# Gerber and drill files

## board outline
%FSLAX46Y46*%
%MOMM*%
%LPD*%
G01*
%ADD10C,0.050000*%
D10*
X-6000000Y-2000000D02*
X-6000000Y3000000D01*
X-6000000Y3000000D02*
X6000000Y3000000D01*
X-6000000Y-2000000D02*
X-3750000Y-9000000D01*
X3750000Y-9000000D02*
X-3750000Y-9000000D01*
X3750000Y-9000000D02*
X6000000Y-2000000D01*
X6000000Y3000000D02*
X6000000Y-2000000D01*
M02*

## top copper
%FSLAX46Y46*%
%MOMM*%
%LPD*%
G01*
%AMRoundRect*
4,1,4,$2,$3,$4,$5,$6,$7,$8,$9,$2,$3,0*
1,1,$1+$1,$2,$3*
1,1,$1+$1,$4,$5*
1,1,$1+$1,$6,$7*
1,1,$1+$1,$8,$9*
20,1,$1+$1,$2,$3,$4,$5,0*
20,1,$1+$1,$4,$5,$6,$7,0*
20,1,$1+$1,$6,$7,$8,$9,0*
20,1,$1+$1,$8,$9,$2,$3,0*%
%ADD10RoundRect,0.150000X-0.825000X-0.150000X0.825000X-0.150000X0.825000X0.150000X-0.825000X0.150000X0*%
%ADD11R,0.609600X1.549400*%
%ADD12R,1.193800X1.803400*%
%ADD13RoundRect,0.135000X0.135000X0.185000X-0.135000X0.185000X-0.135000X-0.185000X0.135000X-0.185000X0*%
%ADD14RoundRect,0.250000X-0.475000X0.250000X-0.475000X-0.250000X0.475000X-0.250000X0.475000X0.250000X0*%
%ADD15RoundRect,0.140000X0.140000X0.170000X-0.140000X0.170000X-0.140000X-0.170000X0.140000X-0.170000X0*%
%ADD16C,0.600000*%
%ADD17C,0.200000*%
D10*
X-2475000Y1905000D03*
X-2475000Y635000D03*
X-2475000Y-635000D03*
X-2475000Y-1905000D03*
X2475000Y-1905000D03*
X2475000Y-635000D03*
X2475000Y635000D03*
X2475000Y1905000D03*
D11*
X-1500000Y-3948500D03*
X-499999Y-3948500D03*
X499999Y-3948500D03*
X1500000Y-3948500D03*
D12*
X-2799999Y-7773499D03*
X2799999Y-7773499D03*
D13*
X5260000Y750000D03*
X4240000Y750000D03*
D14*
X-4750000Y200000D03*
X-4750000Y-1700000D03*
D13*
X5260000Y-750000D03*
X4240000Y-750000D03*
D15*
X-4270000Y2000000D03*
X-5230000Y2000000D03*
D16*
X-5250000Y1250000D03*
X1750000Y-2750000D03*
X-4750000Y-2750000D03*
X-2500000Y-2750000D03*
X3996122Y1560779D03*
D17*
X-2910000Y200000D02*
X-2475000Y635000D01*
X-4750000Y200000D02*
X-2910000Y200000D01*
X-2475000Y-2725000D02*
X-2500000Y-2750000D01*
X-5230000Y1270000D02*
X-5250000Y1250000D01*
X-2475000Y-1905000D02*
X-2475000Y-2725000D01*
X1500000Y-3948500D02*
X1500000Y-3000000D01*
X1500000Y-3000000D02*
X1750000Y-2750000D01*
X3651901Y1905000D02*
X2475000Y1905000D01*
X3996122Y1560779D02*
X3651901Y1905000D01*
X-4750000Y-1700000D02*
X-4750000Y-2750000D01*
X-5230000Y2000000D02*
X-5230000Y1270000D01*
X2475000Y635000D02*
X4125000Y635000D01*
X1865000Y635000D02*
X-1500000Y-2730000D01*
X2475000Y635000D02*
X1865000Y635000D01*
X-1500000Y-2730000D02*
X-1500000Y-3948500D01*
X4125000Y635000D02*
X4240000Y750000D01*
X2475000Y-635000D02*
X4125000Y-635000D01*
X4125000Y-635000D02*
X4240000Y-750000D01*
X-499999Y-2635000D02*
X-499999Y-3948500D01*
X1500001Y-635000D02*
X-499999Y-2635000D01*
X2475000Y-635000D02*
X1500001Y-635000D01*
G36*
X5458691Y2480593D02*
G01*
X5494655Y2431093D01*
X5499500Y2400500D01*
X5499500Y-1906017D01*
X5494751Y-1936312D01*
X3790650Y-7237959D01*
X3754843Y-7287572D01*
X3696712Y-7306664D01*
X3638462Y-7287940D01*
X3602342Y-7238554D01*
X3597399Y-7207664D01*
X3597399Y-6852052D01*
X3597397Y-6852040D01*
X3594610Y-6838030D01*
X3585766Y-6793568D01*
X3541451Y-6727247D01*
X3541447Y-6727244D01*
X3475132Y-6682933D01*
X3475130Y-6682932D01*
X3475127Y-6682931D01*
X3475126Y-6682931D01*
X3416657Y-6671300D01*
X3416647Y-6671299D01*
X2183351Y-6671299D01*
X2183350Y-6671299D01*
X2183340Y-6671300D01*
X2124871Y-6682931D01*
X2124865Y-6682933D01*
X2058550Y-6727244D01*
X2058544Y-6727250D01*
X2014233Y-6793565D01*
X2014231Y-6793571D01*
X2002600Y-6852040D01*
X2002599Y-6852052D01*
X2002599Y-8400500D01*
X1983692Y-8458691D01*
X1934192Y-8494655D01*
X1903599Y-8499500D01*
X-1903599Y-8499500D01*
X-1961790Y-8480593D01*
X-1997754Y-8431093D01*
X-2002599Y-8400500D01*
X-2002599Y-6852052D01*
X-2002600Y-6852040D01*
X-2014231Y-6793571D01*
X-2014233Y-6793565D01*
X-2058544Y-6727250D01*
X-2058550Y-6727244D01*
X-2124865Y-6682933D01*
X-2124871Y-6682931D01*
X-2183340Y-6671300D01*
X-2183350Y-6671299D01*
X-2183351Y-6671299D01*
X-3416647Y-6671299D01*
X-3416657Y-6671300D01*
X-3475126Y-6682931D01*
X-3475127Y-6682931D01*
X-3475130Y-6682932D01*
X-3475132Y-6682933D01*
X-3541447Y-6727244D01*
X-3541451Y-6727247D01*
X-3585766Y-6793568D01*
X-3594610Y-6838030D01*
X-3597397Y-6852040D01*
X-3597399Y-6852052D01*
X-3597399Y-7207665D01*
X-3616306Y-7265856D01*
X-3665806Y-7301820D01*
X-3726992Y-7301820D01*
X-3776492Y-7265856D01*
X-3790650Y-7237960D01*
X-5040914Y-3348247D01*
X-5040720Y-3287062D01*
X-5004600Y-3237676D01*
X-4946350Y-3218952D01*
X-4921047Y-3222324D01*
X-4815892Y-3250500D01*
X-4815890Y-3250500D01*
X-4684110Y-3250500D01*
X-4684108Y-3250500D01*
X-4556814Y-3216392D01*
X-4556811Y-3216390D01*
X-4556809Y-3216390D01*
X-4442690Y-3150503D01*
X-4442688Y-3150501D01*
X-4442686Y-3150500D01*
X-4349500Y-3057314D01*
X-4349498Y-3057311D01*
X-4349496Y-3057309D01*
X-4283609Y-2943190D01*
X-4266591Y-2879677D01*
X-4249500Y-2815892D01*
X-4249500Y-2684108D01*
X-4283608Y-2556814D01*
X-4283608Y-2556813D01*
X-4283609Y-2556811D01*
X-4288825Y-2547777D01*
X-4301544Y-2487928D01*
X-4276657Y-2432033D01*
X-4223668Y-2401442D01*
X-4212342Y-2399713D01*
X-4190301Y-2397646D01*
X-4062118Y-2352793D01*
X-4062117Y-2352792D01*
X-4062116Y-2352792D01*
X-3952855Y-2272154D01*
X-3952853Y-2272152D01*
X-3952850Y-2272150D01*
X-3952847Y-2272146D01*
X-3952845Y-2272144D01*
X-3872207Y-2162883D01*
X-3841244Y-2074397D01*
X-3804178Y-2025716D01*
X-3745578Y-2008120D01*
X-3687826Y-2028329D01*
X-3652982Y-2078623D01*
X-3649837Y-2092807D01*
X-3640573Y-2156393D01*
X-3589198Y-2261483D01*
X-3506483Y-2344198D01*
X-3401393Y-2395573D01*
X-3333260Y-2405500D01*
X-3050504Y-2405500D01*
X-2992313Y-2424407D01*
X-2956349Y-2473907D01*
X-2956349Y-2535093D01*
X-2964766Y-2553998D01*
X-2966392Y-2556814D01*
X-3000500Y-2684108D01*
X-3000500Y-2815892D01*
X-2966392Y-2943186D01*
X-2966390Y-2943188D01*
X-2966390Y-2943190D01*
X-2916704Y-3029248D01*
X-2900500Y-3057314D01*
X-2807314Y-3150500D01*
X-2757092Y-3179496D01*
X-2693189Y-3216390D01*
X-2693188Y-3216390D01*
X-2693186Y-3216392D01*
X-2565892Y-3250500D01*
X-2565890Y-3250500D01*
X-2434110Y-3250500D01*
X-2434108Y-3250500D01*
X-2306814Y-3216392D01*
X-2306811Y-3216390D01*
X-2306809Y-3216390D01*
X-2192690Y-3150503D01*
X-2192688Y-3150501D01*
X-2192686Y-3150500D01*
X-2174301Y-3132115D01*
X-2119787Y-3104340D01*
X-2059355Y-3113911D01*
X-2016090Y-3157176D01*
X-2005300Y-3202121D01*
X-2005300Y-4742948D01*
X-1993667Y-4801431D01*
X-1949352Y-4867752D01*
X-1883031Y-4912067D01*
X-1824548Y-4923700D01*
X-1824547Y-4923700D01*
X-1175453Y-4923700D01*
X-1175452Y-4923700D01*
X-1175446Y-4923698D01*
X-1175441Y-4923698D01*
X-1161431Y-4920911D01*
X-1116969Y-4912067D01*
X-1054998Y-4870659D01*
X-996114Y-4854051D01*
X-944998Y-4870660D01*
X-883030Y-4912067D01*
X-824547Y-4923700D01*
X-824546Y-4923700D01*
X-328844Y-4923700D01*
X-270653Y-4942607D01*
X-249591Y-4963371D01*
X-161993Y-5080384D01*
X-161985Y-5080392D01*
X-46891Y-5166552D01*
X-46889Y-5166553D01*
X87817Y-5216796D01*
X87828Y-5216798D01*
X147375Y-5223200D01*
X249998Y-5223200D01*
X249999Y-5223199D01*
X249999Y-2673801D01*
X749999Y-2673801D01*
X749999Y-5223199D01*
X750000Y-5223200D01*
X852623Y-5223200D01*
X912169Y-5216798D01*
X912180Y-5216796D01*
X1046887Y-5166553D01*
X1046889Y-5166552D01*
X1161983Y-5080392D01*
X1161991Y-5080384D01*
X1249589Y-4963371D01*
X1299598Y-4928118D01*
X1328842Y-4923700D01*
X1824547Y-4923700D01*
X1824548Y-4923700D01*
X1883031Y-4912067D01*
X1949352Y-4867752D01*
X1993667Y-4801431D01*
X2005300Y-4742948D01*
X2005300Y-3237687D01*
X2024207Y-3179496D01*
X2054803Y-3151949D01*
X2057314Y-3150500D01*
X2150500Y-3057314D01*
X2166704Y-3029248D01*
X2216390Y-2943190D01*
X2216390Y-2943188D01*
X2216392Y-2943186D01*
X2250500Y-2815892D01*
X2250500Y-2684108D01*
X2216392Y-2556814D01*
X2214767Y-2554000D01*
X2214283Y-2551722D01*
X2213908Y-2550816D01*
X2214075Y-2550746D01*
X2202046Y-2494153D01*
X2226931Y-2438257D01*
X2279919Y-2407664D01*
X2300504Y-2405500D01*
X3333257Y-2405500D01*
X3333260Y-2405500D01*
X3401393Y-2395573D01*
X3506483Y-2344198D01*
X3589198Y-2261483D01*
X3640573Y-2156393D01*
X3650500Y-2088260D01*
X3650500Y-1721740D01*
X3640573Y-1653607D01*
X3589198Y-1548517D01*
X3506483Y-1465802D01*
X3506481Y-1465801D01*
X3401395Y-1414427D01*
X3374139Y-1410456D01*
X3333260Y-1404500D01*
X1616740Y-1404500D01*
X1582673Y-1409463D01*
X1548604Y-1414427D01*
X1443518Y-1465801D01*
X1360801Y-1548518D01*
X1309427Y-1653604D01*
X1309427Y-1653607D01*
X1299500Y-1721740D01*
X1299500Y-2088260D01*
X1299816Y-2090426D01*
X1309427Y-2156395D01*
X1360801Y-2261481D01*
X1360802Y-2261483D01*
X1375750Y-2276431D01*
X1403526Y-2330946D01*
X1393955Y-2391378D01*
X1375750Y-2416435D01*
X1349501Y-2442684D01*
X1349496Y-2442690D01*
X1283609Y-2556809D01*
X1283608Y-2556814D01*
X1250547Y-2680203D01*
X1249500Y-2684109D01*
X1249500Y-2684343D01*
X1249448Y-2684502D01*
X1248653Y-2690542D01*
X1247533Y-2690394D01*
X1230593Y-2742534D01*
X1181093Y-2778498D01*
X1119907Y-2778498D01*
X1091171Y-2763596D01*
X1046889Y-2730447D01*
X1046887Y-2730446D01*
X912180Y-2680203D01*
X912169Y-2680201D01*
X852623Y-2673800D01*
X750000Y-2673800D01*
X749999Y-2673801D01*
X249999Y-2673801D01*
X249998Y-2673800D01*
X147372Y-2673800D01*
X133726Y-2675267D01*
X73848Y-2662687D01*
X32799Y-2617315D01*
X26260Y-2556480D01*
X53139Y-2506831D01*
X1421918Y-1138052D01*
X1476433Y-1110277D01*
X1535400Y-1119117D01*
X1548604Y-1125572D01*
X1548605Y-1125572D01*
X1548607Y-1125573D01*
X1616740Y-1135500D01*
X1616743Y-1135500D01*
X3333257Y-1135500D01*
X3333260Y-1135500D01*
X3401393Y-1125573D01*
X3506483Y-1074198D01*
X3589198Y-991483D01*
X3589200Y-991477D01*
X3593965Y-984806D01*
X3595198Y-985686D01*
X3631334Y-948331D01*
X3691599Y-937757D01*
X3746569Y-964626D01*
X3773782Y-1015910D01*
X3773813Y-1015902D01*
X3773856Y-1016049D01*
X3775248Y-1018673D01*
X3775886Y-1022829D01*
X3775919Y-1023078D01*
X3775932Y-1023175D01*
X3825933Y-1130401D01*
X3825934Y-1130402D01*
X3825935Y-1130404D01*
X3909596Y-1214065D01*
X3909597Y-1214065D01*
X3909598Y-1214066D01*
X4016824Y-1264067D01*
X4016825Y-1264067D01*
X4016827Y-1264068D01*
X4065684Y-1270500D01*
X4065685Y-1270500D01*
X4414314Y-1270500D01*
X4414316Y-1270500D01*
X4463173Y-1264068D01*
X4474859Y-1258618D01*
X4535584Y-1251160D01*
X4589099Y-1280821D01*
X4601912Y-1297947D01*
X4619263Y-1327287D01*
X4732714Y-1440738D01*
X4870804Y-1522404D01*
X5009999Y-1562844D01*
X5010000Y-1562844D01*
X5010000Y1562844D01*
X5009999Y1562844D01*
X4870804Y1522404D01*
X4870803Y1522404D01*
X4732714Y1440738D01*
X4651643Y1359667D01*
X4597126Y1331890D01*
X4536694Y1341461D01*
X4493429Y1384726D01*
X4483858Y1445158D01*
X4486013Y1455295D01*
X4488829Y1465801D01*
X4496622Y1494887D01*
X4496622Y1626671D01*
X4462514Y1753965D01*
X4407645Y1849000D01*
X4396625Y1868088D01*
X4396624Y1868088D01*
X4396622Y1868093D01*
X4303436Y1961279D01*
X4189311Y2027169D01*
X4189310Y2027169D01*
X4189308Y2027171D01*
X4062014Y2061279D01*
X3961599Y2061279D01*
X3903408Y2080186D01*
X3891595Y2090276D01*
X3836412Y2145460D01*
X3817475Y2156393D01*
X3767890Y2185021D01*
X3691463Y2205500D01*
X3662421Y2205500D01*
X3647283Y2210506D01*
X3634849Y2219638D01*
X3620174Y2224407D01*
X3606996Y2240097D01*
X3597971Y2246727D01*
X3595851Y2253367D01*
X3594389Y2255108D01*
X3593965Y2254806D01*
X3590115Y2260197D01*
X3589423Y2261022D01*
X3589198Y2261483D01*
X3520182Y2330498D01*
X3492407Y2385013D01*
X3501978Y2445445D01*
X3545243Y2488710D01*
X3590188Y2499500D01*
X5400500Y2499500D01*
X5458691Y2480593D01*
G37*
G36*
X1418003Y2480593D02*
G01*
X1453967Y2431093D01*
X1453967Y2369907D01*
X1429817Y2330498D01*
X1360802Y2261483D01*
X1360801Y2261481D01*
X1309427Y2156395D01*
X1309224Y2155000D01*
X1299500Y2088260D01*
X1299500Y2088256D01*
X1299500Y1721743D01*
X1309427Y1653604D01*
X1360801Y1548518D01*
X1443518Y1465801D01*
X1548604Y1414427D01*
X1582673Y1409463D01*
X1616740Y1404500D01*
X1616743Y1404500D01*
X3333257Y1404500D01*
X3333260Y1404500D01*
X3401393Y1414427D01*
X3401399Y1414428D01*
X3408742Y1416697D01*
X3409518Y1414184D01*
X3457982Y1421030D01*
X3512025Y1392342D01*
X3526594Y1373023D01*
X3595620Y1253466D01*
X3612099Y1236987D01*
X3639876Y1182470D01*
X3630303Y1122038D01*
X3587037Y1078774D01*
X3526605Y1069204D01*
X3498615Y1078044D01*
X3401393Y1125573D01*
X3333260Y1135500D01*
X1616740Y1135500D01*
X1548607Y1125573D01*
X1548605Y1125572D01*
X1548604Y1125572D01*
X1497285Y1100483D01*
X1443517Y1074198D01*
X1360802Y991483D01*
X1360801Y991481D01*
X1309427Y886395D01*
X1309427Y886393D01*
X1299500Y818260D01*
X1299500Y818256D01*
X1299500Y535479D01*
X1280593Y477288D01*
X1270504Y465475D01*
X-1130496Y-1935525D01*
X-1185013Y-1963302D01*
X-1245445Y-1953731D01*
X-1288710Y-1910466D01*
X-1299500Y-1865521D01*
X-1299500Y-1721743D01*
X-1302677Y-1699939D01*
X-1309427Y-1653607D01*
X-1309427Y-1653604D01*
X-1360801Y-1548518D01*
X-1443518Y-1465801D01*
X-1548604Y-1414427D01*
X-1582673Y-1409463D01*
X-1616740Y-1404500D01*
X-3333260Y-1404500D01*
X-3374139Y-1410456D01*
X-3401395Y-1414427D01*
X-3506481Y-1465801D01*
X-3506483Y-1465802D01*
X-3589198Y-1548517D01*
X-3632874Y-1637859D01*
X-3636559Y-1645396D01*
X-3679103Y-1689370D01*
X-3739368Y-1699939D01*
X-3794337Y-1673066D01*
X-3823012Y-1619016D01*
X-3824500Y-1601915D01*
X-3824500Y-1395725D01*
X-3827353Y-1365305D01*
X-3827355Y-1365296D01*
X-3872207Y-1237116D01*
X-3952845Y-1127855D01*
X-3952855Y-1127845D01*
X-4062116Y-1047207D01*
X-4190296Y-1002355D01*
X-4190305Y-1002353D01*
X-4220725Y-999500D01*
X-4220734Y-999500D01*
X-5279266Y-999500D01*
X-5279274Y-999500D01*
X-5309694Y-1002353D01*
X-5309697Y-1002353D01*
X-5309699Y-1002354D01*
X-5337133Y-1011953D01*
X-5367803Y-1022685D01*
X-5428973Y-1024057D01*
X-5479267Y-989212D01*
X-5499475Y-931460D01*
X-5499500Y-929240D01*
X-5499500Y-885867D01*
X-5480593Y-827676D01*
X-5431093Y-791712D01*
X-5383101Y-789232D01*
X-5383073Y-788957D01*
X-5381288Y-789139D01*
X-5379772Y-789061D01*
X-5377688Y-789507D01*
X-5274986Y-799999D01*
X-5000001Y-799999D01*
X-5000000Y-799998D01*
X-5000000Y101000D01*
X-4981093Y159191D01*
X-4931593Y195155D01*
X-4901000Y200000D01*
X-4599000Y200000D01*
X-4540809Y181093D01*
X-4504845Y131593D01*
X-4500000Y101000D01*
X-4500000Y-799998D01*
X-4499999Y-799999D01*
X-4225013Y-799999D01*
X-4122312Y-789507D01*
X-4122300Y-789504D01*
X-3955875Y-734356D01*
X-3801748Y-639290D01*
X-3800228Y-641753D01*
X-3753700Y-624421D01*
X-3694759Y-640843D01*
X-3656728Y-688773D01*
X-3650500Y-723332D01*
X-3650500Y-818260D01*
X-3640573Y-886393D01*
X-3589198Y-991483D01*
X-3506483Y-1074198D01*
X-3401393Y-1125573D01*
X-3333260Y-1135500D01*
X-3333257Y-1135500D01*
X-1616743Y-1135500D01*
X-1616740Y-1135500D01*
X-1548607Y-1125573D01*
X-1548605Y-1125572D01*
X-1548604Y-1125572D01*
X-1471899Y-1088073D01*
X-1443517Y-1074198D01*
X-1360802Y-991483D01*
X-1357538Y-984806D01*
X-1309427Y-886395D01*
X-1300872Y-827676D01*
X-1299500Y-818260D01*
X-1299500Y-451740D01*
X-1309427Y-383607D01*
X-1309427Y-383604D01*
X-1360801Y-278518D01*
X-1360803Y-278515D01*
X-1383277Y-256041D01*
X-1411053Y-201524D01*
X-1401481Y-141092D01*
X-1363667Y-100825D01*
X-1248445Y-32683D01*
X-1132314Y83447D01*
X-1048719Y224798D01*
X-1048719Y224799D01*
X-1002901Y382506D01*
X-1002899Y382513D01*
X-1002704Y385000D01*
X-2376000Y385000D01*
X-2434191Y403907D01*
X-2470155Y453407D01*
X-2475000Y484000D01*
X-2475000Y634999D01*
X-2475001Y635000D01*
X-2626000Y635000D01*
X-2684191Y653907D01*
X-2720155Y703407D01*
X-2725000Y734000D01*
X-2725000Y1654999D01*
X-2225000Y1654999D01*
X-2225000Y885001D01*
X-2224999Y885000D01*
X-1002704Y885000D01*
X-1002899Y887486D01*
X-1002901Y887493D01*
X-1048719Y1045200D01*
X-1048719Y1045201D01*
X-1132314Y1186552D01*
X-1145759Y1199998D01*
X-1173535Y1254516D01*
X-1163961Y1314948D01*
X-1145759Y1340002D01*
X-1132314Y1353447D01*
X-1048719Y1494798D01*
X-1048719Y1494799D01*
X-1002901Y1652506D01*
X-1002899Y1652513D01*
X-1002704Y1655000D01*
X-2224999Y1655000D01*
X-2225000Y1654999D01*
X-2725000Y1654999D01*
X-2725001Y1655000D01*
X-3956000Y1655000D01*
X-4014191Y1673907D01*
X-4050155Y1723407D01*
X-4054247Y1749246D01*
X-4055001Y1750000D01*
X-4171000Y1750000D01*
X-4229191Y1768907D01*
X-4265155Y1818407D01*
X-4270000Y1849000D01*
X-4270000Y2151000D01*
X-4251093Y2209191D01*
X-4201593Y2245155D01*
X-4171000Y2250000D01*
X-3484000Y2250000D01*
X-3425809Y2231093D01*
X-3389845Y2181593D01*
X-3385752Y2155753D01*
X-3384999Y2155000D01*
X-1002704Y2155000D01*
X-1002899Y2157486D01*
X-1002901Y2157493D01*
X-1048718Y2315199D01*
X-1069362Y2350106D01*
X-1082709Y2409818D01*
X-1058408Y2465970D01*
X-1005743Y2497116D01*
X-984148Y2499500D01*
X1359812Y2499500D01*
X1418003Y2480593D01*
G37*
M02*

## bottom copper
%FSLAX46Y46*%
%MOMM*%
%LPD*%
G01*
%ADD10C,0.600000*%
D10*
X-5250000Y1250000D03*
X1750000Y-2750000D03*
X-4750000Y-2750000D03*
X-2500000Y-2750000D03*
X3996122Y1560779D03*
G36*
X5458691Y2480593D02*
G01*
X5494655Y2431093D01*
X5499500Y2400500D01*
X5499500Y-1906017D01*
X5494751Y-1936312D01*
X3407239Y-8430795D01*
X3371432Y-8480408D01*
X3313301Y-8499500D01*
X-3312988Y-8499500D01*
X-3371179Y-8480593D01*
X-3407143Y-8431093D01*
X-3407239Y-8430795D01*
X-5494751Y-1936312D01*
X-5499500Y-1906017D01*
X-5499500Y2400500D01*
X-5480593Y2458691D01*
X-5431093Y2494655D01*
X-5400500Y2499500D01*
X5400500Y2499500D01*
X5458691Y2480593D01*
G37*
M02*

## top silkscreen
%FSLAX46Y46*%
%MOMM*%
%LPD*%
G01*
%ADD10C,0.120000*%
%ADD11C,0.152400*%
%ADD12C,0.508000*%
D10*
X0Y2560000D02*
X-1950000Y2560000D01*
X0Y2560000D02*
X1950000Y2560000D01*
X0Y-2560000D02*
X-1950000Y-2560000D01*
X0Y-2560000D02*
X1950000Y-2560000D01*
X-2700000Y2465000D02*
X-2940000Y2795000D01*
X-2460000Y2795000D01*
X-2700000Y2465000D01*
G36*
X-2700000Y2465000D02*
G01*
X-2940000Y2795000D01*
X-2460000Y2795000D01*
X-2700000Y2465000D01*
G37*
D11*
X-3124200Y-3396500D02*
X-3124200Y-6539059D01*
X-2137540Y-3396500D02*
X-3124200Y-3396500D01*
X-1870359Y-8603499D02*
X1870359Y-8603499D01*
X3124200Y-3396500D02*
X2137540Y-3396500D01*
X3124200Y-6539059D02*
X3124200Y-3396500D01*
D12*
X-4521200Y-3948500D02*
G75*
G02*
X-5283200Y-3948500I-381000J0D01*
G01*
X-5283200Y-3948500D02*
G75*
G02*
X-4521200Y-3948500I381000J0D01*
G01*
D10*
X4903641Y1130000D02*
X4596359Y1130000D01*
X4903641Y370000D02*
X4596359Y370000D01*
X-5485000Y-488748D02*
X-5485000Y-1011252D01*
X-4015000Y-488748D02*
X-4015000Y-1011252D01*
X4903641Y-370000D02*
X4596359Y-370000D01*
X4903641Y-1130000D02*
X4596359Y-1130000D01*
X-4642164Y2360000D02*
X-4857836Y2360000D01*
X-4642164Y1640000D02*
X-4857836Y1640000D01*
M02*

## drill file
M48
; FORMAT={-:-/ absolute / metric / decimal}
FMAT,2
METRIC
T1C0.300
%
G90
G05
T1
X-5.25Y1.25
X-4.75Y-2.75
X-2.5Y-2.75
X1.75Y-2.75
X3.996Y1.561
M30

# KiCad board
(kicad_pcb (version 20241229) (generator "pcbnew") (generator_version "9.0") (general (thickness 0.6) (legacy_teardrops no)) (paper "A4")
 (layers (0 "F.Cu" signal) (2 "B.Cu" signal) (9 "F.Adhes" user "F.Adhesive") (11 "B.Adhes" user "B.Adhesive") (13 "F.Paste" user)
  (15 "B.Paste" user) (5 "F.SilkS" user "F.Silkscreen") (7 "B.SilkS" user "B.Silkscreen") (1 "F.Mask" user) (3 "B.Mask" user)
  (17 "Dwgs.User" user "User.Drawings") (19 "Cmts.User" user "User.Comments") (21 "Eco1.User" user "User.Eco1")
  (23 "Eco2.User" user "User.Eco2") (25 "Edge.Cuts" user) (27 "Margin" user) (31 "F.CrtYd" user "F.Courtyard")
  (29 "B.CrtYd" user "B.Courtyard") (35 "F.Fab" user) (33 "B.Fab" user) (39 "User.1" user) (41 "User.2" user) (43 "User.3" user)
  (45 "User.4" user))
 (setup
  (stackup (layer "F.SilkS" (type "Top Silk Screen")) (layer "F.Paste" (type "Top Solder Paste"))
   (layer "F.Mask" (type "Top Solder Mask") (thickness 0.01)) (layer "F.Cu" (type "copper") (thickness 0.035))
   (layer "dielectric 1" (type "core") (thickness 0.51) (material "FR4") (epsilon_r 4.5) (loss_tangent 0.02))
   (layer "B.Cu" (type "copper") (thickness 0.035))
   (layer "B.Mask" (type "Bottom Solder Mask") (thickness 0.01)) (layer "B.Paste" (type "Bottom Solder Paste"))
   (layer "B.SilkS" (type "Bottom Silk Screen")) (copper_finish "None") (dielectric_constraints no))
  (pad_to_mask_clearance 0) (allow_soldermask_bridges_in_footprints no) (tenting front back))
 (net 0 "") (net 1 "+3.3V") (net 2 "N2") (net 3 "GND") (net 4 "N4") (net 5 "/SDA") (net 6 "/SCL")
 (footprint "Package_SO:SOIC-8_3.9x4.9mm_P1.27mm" (layer "F.Cu") (at 0 0)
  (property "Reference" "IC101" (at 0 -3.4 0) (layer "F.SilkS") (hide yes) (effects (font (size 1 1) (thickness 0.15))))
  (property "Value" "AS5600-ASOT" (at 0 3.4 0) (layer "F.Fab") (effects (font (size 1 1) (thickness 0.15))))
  (fp_line (start 0 -2.56) (end -1.95 -2.56) (stroke (width 0.12) (type solid)) (layer "F.SilkS"))
  (fp_line (start 0 -2.56) (end 1.95 -2.56) (stroke (width 0.12) (type solid)) (layer "F.SilkS"))
  (fp_line (start 0 2.56) (end -1.95 2.56) (stroke (width 0.12) (type solid)) (layer "F.SilkS"))
  (fp_line (start 0 2.56) (end 1.95 2.56) (stroke (width 0.12) (type solid)) (layer "F.SilkS"))
  (fp_poly (pts (xy -2.7 -2.465) (xy -2.94 -2.795) (xy -2.46 -2.795)) (stroke (width 0.12) (type solid)) (fill yes) (layer "F.SilkS"))
  (pad "1" smd roundrect (at -2.475 -1.905) (size 1.95 0.6) (layers "F.Cu" "F.Mask" "F.Paste") (roundrect_rratio 0.25) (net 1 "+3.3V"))
  (pad "2" smd roundrect (at -2.475 -0.635) (size 1.95 0.6) (layers "F.Cu" "F.Mask" "F.Paste") (roundrect_rratio 0.25) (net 1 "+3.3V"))
  (pad "3" smd roundrect (at -2.475 0.635) (size 1.95 0.6) (layers "F.Cu" "F.Mask" "F.Paste") (roundrect_rratio 0.25) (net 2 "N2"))
  (pad "4" smd roundrect (at -2.475 1.905) (size 1.95 0.6) (layers "F.Cu" "F.Mask" "F.Paste") (roundrect_rratio 0.25) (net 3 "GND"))
  (pad "5" smd roundrect (at 2.475 1.905) (size 1.95 0.6) (layers "F.Cu" "F.Mask" "F.Paste") (roundrect_rratio 0.25) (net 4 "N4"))
  (pad "6" smd roundrect (at 2.475 0.635) (size 1.95 0.6) (layers "F.Cu" "F.Mask" "F.Paste") (roundrect_rratio 0.25) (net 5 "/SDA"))
  (pad "7" smd roundrect (at 2.475 -0.635) (size 1.95 0.6) (layers "F.Cu" "F.Mask" "F.Paste") (roundrect_rratio 0.25) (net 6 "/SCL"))
  (pad "8" smd roundrect (at 2.475 -1.905) (size 1.95 0.6) (layers "F.Cu" "F.Mask" "F.Paste") (roundrect_rratio 0.25) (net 3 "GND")))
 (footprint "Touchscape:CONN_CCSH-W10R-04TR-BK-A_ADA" (layer "F.Cu") (at 0 6)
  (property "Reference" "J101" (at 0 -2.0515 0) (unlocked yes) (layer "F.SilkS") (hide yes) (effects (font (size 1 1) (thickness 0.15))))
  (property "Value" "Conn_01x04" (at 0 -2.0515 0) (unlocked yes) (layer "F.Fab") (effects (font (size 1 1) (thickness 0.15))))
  (fp_line (start -3.1242 -2.6035) (end -3.1242 0.539059) (stroke (width 0.1524) (type solid)) (layer "F.SilkS"))
  (fp_line (start -2.13754 -2.6035) (end -3.1242 -2.6035) (stroke (width 0.1524) (type solid)) (layer "F.SilkS"))
  (fp_line (start -1.870359 2.603499) (end 1.870359 2.603499) (stroke (width 0.1524) (type solid)) (layer "F.SilkS"))
  (fp_line (start 3.1242 -2.6035) (end 2.13754 -2.6035) (stroke (width 0.1524) (type solid)) (layer "F.SilkS"))
  (fp_line (start 3.1242 0.539059) (end 3.1242 -2.6035) (stroke (width 0.1524) (type solid)) (layer "F.SilkS"))
  (fp_circle (center -4.9022 -2.0515) (end -4.5212 -2.0515) (stroke (width 0.508) (type solid)) (fill no) (layer "F.SilkS"))
  (pad "1" smd rect (at -1.5 -2.0515) (size 0.6096 1.5494) (layers "F.Cu" "F.Mask" "F.Paste") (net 6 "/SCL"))
  (pad "2" smd rect (at -0.499999 -2.0515) (size 0.6096 1.5494) (layers "F.Cu" "F.Mask" "F.Paste") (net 5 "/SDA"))
  (pad "3" smd rect (at 0.499999 -2.0515) (size 0.6096 1.5494) (layers "F.Cu" "F.Mask" "F.Paste") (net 1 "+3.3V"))
  (pad "4" smd rect (at 1.5 -2.0515) (size 0.6096 1.5494) (layers "F.Cu" "F.Mask" "F.Paste") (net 3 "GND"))
  (pad "5" smd rect (at -2.799999 1.773499) (size 1.1938 1.8034) (layers "F.Cu" "F.Mask" "F.Paste"))
  (pad "6" smd rect (at 2.799999 1.773499) (size 1.1938 1.8034) (layers "F.Cu" "F.Mask" "F.Paste")))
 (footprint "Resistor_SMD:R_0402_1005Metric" (layer "F.Cu") (at 4.75 -0.75 180)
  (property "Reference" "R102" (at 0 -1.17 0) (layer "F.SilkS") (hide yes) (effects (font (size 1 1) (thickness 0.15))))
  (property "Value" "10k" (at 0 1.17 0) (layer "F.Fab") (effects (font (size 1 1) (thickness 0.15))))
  (fp_line (start -0.153641 0.38) (end 0.153641 0.38) (stroke (width 0.12) (type solid)) (layer "F.SilkS"))
  (fp_line (start -0.153641 -0.38) (end 0.153641 -0.38) (stroke (width 0.12) (type solid)) (layer "F.SilkS"))
  (pad "1" smd roundrect (at -0.51 0 180) (size 0.54 0.64) (layers "F.Cu" "F.Mask" "F.Paste") (roundrect_rratio 0.25) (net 1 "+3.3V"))
  (pad "2" smd roundrect (at 0.51 0 180) (size 0.54 0.64) (layers "F.Cu" "F.Mask" "F.Paste") (roundrect_rratio 0.25) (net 6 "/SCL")))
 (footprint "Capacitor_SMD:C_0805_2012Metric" (layer "F.Cu") (at -4.75 0.75 -90)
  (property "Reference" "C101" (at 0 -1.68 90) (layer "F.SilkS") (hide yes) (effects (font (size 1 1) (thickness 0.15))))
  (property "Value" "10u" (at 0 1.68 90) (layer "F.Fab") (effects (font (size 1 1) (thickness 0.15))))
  (fp_line (start -0.261252 0.735) (end 0.261252 0.735) (stroke (width 0.12) (type solid)) (layer "F.SilkS"))
  (fp_line (start -0.261252 -0.735) (end 0.261252 -0.735) (stroke (width 0.12) (type solid)) (layer "F.SilkS"))
  (pad "1" smd roundrect (at -0.95 0 270) (size 1 1.45) (layers "F.Cu" "F.Mask" "F.Paste") (roundrect_rratio 0.25) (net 1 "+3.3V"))
  (pad "2" smd roundrect (at 0.95 0 270) (size 1 1.45) (layers "F.Cu" "F.Mask" "F.Paste") (roundrect_rratio 0.25) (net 3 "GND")))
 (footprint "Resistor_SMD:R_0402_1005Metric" (layer "F.Cu") (at 4.75 0.75 180)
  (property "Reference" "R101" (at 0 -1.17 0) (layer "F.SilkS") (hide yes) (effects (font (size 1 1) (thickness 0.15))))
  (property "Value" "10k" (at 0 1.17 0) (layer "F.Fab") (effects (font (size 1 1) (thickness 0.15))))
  (fp_line (start -0.153641 0.38) (end 0.153641 0.38) (stroke (width 0.12) (type solid)) (layer "F.SilkS"))
  (fp_line (start -0.153641 -0.38) (end 0.153641 -0.38) (stroke (width 0.12) (type solid)) (layer "F.SilkS"))
  (pad "1" smd roundrect (at -0.51 0 180) (size 0.54 0.64) (layers "F.Cu" "F.Mask" "F.Paste") (roundrect_rratio 0.25) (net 1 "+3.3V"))
  (pad "2" smd roundrect (at 0.51 0 180) (size 0.54 0.64) (layers "F.Cu" "F.Mask" "F.Paste") (roundrect_rratio 0.25) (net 5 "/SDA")))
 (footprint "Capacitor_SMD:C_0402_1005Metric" (layer "F.Cu") (at -4.75 -2 180)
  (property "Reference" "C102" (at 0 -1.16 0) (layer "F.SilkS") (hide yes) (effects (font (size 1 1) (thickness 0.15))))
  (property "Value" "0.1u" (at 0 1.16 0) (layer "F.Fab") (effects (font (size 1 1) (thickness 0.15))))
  (fp_line (start -0.107836 0.36) (end 0.107836 0.36) (stroke (width 0.12) (type solid)) (layer "F.SilkS"))
  (fp_line (start -0.107836 -0.36) (end 0.107836 -0.36) (stroke (width 0.12) (type solid)) (layer "F.SilkS"))
  (pad "1" smd roundrect (at -0.48 0 180) (size 0.56 0.62) (layers "F.Cu" "F.Mask" "F.Paste") (roundrect_rratio 0.25) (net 1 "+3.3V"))
  (pad "2" smd roundrect (at 0.48 0 180) (size 0.56 0.62) (layers "F.Cu" "F.Mask" "F.Paste") (roundrect_rratio 0.25) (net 3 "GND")))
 (gr_line (start -6 2) (end -6 -3) (stroke (width 0.05) (type default)) (layer "Edge.Cuts"))
 (gr_line (start -6 -3) (end 6 -3) (stroke (width 0.05) (type default)) (layer "Edge.Cuts"))
 (gr_line (start -6 2) (end -3.75 9) (stroke (width 0.05) (type default)) (layer "Edge.Cuts"))
 (gr_line (start 3.75 9) (end -3.75 9) (stroke (width 0.05) (type default)) (layer "Edge.Cuts"))
 (gr_line (start 3.75 9) (end 6 2) (stroke (width 0.05) (type default)) (layer "Edge.Cuts"))
 (gr_line (start 6 -3) (end 6 2) (stroke (width 0.05) (type default)) (layer "Edge.Cuts"))
 (segment (start -2.91 -0.2) (end -2.475 -0.635) (width 0.2) (layer "F.Cu") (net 1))
 (segment (start -4.75 -0.2) (end -2.91 -0.2) (width 0.2) (layer "F.Cu") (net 1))
 (segment (start -2.475 2.725) (end -2.5 2.75) (width 0.2) (layer "F.Cu") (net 3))
 (segment (start -5.23 -1.27) (end -5.25 -1.25) (width 0.2) (layer "F.Cu") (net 3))
 (segment (start -2.475 1.905) (end -2.475 2.725) (width 0.2) (layer "F.Cu") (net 3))
 (segment (start 1.5 3.9485) (end 1.5 3) (width 0.2) (layer "F.Cu") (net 3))
 (segment (start 1.5 3) (end 1.75 2.75) (width 0.2) (layer "F.Cu") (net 3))
 (segment (start 3.651901 -1.905) (end 2.475 -1.905) (width 0.2) (layer "F.Cu") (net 3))
 (segment (start 3.996122 -1.560779) (end 3.651901 -1.905) (width 0.2) (layer "F.Cu") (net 3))
 (segment (start -4.75 1.7) (end -4.75 2.75) (width 0.2) (layer "F.Cu") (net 3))
 (segment (start -5.23 -2) (end -5.23 -1.27) (width 0.2) (layer "F.Cu") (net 3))
 (via (at -5.25 -1.25) (size 0.6) (drill 0.3) (layers "F.Cu" "B.Cu") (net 3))
 (via (at 1.75 2.75) (size 0.6) (drill 0.3) (layers "F.Cu" "B.Cu") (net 3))
 (via (at -4.75 2.75) (size 0.6) (drill 0.3) (layers "F.Cu" "B.Cu") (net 3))
 (via (at -2.5 2.75) (size 0.6) (drill 0.3) (layers "F.Cu" "B.Cu") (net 3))
 (via (at 3.996122 -1.560779) (size 0.6) (drill 0.3) (layers "F.Cu" "B.Cu") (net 3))
 (segment (start 2.475 -0.635) (end 4.125 -0.635) (width 0.2) (layer "F.Cu") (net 6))
 (segment (start 1.865 -0.635) (end -1.5 2.73) (width 0.2) (layer "F.Cu") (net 6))
 (segment (start 2.475 -0.635) (end 1.865 -0.635) (width 0.2) (layer "F.Cu") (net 6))
 (segment (start -1.5 2.73) (end -1.5 3.9485) (width 0.2) (layer "F.Cu") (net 6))
 (segment (start 4.125 -0.635) (end 4.24 -0.75) (width 0.2) (layer "F.Cu") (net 6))
 (segment (start 2.475 0.635) (end 4.125 0.635) (width 0.2) (layer "F.Cu") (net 5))
 (segment (start 4.125 0.635) (end 4.24 0.75) (width 0.2) (layer "F.Cu") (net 5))
 (segment (start -0.499999 2.635) (end -0.499999 3.9485) (width 0.2) (layer "F.Cu") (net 5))
 (segment (start 1.500001 0.635) (end -0.499999 2.635) (width 0.2) (layer "F.Cu") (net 5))
 (segment (start 2.475 0.635) (end 1.500001 0.635) (width 0.2) (layer "F.Cu") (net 5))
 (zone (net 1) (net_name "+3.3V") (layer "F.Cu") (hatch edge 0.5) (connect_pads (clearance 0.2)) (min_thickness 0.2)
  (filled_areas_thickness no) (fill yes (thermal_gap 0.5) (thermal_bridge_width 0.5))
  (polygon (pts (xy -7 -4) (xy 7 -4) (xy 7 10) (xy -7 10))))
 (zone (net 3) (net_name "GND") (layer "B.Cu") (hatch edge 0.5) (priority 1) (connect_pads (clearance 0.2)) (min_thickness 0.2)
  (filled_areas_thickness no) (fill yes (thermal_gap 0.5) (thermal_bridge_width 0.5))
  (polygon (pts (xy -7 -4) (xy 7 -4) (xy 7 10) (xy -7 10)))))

